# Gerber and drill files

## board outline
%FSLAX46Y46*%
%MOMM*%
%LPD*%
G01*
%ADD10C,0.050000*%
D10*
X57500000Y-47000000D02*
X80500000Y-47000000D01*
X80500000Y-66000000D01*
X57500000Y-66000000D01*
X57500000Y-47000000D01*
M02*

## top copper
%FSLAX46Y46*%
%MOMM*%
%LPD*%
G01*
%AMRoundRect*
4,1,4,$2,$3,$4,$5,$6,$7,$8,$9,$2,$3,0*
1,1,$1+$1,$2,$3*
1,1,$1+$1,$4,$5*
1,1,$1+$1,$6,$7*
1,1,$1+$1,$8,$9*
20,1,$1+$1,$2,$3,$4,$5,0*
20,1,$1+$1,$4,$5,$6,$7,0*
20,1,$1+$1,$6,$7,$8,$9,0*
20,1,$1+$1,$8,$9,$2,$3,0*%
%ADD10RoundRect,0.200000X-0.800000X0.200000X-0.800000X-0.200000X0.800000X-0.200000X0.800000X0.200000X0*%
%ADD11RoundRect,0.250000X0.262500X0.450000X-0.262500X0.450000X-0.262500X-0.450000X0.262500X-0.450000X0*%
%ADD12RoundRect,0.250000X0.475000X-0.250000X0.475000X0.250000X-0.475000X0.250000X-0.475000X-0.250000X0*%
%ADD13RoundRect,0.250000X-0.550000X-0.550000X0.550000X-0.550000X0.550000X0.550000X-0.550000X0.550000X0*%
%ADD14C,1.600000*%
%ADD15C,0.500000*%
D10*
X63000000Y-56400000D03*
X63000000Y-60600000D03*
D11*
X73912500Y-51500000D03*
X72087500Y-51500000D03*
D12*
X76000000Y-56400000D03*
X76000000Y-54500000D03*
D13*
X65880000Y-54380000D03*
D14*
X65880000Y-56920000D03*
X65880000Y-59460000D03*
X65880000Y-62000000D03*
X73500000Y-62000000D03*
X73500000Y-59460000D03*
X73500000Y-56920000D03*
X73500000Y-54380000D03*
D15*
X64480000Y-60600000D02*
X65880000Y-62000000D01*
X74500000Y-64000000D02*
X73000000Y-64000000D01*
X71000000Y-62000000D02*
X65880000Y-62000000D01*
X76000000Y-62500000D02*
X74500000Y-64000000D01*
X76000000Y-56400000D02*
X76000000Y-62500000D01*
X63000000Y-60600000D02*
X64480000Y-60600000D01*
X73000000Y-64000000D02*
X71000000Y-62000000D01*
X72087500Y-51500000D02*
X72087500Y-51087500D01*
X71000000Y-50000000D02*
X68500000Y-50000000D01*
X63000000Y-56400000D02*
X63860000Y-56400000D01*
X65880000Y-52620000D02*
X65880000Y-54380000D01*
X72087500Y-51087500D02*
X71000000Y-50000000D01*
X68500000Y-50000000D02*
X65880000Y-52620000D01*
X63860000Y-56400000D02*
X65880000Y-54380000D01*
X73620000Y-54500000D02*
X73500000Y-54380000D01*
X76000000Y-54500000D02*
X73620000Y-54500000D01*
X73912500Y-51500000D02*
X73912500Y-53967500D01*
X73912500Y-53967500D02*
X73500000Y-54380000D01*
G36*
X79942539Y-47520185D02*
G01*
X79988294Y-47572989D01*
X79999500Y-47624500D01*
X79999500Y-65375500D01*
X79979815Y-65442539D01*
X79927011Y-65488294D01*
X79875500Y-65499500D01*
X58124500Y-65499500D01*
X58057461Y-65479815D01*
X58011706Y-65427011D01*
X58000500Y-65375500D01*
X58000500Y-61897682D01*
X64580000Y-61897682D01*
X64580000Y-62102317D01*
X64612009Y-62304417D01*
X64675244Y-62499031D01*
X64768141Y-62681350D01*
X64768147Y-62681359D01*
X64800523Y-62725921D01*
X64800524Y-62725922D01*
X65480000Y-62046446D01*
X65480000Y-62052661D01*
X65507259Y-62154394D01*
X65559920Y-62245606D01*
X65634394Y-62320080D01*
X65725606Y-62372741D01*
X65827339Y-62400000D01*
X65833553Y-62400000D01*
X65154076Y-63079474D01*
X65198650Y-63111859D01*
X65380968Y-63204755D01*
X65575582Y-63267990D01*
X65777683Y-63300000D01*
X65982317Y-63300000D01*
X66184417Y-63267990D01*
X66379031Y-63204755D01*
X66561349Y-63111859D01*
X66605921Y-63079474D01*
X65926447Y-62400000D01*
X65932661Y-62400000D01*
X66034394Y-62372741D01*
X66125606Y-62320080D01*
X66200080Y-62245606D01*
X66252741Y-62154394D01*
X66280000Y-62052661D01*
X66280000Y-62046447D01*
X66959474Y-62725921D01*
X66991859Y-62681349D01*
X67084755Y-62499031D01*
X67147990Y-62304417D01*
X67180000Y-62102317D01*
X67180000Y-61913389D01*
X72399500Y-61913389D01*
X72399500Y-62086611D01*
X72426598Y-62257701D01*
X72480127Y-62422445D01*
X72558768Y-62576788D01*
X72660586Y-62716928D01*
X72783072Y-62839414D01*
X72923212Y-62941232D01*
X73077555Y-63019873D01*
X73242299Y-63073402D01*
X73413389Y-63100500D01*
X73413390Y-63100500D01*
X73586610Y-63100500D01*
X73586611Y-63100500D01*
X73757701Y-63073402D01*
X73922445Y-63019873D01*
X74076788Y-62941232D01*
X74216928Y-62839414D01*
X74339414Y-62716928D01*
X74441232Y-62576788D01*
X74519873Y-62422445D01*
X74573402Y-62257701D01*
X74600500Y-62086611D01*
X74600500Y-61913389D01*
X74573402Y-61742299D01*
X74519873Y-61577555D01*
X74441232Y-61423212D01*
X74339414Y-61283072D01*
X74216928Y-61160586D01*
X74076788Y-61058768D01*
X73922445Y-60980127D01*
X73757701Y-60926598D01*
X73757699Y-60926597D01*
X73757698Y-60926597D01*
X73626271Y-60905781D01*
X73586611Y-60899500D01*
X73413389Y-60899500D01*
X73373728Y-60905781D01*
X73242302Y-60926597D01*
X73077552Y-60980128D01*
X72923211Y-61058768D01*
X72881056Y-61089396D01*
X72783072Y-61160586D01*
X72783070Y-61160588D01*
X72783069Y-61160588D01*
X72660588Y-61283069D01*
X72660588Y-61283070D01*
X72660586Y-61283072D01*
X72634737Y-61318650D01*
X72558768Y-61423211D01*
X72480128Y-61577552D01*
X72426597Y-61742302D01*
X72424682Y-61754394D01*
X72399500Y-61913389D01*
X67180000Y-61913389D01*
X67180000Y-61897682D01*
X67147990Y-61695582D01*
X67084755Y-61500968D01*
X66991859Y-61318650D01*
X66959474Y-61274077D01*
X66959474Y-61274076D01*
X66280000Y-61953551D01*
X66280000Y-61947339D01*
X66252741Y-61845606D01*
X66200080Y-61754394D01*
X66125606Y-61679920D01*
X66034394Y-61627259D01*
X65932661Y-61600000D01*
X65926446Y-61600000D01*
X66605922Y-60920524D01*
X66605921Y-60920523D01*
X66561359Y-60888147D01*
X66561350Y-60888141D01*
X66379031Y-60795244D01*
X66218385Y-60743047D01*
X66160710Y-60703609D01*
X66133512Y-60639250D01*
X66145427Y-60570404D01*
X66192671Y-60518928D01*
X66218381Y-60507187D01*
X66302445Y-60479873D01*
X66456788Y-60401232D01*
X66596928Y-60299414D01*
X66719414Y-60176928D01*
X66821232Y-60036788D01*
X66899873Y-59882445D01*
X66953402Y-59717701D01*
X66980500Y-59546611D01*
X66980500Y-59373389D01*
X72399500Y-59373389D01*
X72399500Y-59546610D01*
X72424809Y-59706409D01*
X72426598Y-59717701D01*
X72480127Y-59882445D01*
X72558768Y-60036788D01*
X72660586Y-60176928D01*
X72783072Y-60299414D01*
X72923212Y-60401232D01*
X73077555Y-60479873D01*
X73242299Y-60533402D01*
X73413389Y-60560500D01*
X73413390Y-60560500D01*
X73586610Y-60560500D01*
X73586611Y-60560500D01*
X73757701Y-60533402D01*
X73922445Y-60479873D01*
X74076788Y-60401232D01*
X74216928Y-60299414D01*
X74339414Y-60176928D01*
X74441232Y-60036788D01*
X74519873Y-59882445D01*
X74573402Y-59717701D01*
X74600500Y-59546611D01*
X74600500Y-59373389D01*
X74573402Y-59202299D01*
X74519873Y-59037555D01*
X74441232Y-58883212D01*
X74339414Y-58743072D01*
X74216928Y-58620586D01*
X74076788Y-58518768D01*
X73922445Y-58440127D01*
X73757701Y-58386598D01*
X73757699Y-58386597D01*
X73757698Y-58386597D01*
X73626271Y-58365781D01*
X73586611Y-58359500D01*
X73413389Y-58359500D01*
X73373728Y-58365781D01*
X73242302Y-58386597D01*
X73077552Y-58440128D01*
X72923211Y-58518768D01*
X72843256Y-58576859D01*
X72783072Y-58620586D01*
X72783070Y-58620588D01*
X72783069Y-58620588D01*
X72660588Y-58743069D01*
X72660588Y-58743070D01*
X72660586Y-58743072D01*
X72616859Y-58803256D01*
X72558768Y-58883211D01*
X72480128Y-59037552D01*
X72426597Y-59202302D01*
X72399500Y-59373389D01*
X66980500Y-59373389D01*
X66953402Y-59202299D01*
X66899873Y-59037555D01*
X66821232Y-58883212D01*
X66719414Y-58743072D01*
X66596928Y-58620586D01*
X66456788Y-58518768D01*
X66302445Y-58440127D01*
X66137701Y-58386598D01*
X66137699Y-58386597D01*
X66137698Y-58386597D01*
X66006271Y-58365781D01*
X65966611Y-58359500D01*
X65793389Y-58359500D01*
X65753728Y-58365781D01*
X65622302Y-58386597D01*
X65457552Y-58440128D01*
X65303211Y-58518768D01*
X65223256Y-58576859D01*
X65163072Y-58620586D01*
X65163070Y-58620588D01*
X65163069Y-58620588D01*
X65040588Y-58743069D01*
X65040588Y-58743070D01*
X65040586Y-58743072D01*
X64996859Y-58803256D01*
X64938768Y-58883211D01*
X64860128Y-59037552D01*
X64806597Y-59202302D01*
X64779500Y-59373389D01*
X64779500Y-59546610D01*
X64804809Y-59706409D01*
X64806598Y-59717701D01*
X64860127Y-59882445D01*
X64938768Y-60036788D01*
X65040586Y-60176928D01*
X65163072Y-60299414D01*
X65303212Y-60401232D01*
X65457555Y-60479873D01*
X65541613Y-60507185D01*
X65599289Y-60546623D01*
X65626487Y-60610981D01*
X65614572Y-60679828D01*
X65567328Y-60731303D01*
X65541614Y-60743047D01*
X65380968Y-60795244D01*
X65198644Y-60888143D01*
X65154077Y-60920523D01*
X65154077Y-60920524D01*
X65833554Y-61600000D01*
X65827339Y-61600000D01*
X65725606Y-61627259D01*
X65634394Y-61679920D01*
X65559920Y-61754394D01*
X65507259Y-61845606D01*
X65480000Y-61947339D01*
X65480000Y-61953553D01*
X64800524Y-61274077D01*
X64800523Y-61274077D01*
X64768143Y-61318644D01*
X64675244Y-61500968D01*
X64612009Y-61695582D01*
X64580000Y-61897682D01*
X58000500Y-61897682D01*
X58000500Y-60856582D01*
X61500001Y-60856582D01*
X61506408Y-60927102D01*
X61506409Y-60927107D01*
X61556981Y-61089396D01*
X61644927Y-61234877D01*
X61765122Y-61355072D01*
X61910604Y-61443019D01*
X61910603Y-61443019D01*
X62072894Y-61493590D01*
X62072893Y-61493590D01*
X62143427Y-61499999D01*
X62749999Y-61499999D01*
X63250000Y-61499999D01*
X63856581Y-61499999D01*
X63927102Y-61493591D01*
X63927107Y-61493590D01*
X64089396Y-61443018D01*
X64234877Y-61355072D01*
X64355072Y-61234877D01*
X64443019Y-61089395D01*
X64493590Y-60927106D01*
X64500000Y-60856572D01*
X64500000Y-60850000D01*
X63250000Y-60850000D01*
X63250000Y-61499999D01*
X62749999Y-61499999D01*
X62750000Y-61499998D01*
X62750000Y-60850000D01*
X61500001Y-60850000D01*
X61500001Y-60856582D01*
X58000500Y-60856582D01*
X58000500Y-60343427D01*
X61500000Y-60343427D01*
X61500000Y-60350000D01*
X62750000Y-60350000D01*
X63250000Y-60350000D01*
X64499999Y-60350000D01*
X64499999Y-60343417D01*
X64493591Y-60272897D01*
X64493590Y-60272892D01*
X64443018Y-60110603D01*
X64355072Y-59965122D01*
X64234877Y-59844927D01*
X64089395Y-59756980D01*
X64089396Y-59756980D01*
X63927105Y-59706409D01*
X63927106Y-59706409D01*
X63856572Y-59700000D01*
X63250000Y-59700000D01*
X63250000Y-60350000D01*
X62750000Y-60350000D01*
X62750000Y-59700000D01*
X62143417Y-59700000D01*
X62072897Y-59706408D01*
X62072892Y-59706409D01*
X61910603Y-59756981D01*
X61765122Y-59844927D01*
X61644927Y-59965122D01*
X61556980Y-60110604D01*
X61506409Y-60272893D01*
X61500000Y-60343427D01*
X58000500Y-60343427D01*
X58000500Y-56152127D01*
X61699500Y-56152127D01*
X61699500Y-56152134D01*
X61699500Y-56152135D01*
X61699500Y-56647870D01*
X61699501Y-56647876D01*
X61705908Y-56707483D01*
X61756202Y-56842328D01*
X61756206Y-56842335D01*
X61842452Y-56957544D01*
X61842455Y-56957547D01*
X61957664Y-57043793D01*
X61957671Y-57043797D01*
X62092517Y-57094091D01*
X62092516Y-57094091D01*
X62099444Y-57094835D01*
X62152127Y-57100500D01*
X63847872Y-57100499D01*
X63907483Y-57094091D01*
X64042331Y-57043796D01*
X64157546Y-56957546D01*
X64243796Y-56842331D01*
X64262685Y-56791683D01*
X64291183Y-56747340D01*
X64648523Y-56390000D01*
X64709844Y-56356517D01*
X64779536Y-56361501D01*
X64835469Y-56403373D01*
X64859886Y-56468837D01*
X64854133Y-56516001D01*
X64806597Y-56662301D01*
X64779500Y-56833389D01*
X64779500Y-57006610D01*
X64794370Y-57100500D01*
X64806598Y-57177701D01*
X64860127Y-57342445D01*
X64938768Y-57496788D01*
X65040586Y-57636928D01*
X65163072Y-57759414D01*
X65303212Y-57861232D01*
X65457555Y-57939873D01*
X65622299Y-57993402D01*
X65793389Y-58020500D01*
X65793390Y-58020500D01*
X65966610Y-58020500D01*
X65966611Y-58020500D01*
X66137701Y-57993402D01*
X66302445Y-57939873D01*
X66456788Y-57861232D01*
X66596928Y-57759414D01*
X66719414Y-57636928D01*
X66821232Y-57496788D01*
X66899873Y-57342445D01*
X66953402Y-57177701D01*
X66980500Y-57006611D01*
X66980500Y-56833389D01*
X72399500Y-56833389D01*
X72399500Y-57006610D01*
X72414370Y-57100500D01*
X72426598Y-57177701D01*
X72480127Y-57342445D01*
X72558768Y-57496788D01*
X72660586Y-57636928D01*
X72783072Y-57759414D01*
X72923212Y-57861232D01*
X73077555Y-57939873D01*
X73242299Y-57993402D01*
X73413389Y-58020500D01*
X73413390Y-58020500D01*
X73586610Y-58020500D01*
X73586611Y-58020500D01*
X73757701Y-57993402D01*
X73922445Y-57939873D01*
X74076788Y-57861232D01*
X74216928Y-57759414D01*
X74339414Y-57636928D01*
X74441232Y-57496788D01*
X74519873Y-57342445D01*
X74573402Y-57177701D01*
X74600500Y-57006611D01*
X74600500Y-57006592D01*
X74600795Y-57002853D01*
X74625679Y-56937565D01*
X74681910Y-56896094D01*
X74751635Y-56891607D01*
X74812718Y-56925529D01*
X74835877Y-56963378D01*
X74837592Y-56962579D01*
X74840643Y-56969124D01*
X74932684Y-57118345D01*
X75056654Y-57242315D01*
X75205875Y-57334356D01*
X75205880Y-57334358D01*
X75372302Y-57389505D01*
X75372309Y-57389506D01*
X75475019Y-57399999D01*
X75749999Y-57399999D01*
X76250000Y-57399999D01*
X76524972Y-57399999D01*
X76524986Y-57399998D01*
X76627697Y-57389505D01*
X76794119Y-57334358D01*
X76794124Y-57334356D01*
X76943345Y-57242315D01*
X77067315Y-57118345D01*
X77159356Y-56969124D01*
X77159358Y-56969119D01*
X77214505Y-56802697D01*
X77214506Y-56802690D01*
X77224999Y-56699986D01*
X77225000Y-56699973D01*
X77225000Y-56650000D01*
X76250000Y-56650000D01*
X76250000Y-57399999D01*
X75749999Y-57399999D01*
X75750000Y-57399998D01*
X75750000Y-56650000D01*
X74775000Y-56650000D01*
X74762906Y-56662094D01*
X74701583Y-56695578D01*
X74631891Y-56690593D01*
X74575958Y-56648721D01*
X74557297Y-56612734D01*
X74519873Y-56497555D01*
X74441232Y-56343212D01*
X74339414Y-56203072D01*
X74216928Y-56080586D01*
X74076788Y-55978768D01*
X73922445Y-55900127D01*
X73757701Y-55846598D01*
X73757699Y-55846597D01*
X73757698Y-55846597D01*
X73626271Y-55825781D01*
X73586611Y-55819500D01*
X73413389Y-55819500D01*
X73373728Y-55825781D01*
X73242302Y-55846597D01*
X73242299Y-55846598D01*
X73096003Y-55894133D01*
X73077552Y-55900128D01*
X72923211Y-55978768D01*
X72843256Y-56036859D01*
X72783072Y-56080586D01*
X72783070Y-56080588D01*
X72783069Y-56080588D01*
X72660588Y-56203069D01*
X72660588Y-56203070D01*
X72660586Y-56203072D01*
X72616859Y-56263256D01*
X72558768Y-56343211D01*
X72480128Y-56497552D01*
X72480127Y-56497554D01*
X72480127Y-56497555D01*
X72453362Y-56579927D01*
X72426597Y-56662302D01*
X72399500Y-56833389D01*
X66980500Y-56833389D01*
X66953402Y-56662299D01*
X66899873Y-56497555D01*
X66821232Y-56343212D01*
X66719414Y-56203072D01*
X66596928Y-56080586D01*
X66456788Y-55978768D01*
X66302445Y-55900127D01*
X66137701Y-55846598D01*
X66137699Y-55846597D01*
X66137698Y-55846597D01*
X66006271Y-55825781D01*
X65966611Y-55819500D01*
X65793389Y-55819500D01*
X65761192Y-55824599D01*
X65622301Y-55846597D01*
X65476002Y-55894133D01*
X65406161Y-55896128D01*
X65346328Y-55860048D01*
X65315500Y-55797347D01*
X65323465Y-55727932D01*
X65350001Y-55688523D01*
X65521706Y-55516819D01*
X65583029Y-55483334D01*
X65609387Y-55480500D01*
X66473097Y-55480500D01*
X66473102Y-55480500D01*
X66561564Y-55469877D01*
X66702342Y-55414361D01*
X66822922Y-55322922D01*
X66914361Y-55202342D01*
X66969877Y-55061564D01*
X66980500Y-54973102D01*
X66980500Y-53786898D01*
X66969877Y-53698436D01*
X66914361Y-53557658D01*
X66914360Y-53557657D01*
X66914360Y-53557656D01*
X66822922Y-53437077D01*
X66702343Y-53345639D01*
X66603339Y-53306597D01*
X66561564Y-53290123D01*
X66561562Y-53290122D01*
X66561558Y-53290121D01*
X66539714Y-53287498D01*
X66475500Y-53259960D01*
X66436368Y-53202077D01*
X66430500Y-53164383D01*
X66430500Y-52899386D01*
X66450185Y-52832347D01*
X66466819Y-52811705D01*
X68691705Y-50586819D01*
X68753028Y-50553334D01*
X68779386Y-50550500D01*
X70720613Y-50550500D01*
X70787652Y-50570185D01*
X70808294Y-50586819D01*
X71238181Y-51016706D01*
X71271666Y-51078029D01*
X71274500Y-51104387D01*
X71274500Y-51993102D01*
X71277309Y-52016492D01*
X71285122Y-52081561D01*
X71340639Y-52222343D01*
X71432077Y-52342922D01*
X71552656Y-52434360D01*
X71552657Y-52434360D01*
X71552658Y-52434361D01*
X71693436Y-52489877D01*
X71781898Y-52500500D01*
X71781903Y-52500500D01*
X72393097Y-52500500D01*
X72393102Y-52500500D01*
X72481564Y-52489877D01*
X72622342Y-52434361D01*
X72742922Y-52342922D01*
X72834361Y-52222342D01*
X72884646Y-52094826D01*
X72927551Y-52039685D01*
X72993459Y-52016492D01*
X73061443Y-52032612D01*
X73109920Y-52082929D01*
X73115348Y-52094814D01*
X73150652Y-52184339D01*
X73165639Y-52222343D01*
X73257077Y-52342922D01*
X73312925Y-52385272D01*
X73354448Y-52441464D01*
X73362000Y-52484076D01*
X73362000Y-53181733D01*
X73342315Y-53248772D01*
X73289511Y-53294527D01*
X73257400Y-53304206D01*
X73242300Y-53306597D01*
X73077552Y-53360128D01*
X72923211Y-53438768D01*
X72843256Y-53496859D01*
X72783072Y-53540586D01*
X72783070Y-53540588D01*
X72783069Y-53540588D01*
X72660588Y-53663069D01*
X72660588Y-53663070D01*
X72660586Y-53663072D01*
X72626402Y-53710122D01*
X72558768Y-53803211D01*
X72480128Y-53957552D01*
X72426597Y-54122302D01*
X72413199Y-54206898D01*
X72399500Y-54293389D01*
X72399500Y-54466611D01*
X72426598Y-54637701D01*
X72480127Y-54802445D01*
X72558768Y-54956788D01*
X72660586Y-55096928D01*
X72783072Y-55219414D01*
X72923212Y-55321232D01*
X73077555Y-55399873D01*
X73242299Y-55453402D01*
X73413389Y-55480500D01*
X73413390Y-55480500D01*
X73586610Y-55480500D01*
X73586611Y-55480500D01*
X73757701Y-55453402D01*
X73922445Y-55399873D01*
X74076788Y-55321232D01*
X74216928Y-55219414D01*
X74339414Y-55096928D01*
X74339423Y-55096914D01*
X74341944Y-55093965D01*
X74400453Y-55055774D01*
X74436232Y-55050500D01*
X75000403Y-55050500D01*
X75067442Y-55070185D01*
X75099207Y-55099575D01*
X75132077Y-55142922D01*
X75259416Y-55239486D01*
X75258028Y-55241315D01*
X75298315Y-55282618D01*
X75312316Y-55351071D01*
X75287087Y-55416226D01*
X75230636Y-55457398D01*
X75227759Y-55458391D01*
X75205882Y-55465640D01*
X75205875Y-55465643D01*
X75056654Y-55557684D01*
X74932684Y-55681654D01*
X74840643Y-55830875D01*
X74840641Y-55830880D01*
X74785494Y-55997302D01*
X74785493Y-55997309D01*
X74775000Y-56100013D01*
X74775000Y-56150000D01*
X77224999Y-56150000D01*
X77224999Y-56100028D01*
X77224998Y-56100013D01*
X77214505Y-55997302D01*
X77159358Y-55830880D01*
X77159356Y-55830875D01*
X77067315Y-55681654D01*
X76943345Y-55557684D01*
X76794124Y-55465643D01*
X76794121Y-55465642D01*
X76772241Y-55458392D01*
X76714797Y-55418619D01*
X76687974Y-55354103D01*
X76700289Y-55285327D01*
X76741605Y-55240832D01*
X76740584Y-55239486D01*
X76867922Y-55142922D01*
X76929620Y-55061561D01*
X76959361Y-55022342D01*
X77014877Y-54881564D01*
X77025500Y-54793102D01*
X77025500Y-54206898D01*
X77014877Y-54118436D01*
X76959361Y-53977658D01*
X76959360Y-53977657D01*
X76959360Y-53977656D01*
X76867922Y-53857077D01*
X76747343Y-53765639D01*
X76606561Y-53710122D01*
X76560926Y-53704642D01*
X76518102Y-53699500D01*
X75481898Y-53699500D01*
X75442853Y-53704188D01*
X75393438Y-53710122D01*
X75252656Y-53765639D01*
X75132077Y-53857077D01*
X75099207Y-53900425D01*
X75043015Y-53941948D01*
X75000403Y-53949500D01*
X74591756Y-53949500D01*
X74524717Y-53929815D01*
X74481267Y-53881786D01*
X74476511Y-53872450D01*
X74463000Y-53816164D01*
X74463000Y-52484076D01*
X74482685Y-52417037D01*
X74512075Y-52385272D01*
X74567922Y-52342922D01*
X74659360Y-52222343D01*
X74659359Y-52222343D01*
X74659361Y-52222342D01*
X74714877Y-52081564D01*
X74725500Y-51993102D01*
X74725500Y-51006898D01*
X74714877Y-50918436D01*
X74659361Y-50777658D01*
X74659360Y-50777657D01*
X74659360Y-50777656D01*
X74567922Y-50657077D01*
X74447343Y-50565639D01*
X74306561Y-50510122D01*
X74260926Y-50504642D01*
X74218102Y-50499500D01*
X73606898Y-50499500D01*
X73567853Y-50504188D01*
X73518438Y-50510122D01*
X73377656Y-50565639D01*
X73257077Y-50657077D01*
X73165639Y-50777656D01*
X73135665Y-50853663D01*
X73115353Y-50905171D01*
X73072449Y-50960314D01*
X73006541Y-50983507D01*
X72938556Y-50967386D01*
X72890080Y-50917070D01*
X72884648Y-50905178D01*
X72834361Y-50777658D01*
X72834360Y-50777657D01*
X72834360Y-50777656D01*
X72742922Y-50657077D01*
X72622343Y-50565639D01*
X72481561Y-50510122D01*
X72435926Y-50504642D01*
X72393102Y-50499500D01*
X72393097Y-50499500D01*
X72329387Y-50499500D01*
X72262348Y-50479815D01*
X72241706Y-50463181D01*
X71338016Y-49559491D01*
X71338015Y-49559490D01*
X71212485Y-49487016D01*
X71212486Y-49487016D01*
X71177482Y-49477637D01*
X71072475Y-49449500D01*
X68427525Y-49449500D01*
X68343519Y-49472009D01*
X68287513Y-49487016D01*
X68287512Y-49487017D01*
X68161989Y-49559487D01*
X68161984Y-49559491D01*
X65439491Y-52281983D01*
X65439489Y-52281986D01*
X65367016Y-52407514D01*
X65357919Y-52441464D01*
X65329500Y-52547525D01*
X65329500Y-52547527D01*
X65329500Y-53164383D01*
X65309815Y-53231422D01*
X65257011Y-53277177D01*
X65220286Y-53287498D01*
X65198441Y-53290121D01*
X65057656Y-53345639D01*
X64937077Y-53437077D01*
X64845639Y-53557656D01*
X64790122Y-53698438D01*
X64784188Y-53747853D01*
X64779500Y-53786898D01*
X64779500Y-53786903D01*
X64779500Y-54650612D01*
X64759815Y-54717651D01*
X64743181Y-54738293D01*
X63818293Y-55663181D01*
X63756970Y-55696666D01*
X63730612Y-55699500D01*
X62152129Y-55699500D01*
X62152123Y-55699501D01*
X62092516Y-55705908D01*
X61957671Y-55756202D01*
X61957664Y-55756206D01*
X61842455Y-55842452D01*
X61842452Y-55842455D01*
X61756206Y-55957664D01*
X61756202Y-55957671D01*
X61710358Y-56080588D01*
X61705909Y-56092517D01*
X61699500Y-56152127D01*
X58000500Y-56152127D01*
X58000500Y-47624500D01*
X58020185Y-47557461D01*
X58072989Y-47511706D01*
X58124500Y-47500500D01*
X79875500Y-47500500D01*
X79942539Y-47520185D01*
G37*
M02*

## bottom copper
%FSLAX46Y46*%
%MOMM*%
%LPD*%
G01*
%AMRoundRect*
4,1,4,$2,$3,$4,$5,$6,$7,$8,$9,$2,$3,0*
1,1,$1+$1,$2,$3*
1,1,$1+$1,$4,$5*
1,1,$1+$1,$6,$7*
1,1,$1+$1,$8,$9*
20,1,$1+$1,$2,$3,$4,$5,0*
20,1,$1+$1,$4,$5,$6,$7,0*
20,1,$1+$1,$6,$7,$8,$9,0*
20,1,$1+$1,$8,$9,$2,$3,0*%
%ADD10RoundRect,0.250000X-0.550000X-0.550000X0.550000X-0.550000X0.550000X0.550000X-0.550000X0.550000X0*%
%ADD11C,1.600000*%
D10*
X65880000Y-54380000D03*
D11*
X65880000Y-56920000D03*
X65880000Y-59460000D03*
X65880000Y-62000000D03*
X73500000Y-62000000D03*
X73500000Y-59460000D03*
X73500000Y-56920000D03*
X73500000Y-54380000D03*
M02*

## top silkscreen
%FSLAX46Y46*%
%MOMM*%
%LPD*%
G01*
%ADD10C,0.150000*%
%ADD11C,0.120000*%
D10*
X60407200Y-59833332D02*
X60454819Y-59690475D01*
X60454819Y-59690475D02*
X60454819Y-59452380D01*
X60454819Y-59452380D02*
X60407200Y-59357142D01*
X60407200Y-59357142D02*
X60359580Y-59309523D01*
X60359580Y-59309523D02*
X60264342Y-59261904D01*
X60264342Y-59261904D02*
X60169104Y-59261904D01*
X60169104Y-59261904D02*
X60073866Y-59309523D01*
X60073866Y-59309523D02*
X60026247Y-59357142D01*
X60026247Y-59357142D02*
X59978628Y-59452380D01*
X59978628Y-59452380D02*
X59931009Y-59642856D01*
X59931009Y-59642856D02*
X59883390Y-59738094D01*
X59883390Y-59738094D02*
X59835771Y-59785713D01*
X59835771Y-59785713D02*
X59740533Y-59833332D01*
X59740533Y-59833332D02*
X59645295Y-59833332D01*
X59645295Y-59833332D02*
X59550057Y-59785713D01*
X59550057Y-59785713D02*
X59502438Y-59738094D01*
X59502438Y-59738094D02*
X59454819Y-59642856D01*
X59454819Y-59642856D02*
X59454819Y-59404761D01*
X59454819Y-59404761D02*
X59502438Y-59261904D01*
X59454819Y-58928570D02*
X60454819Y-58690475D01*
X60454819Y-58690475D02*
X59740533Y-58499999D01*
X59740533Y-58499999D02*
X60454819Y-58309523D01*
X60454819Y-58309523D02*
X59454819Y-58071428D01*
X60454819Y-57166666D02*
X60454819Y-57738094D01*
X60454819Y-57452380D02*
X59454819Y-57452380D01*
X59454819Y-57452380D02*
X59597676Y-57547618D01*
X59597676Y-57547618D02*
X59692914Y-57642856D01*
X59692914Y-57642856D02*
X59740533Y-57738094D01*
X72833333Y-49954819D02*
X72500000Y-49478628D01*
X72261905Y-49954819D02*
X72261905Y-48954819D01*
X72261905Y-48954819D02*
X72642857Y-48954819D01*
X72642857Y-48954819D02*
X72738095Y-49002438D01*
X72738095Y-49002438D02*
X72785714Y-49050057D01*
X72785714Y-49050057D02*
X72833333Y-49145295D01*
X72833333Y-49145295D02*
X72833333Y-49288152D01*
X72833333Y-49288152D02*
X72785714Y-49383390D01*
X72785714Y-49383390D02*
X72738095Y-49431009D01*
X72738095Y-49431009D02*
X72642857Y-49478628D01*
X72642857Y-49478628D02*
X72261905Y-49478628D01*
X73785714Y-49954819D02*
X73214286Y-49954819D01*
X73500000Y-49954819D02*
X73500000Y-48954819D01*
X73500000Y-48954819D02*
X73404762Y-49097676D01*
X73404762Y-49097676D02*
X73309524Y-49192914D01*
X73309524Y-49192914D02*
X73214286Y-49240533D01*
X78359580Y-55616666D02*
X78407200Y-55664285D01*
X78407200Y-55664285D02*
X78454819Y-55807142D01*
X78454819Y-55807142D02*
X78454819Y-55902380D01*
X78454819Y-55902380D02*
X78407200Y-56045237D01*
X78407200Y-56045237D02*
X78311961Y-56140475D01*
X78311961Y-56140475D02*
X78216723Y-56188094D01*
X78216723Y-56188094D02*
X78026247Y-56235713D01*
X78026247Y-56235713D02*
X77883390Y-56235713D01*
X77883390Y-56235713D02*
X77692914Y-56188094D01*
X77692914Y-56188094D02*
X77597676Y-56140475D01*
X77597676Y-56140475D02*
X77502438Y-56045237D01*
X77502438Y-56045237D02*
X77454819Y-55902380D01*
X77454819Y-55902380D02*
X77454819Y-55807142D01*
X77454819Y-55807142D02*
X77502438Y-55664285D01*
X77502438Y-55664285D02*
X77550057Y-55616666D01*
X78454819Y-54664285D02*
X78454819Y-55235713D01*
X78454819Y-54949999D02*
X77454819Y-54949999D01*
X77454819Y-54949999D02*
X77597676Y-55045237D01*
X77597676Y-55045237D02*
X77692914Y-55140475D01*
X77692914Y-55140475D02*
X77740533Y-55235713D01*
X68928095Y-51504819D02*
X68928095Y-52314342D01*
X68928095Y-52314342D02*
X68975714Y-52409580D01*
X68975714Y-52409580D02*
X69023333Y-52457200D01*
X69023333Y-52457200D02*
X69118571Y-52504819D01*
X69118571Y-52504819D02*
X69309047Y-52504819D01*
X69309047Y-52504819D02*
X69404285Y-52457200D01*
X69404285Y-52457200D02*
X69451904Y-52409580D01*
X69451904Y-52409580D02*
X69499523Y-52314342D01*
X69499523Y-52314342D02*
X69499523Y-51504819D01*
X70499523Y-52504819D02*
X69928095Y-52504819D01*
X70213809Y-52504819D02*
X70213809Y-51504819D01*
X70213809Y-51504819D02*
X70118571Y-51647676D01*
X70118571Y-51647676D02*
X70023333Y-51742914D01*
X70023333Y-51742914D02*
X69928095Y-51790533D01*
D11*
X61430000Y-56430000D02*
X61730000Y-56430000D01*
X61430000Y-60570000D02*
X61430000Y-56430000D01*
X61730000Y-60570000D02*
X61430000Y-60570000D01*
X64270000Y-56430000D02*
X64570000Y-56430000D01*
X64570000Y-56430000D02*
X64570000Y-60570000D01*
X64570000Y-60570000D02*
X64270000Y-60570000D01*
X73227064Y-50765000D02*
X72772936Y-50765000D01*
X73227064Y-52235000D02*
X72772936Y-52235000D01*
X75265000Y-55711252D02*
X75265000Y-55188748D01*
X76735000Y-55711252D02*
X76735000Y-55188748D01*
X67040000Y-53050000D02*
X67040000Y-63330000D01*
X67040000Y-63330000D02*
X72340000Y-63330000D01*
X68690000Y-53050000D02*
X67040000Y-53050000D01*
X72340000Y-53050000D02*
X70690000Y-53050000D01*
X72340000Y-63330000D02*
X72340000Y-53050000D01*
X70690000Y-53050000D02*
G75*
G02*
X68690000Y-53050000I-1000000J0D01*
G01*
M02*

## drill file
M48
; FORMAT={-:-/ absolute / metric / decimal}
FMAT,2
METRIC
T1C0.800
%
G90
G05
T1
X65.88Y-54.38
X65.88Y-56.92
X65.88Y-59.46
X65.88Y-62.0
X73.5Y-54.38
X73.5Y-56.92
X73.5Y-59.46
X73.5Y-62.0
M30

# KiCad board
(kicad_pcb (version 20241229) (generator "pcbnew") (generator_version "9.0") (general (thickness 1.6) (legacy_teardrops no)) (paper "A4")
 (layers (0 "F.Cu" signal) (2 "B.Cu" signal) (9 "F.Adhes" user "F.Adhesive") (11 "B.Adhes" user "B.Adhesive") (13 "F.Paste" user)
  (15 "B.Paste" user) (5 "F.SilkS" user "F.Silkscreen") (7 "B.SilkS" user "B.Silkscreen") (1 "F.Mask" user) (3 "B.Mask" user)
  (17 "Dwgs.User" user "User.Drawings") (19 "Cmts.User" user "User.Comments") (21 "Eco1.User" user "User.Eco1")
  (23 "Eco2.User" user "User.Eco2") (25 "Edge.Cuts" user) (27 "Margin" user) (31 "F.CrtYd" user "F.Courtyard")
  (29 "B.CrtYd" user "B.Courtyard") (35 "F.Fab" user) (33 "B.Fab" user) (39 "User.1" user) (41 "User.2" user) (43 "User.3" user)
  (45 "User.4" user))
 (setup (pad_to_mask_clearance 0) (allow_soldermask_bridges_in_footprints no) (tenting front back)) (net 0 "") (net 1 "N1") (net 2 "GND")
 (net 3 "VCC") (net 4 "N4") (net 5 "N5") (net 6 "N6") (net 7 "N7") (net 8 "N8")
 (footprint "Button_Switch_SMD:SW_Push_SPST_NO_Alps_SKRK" (layer "F.Cu") (at 63 58.5 -90)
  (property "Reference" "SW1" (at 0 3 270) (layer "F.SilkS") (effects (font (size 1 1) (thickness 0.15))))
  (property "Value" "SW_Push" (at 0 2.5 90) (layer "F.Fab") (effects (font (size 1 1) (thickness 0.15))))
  (fp_line (start -2.07 1.57) (end -2.07 1.27) (stroke (width 0.12) (type solid)) (layer "F.SilkS"))
  (fp_line (start 2.07 1.57) (end -2.07 1.57) (stroke (width 0.12) (type solid)) (layer "F.SilkS"))
  (fp_line (start 2.07 1.27) (end 2.07 1.57) (stroke (width 0.12) (type solid)) (layer "F.SilkS"))
  (fp_line (start -2.07 -1.27) (end -2.07 -1.57) (stroke (width 0.12) (type solid)) (layer "F.SilkS"))
  (fp_line (start -2.07 -1.57) (end 2.07 -1.57) (stroke (width 0.12) (type solid)) (layer "F.SilkS"))
  (fp_line (start 2.07 -1.57) (end 2.07 -1.27) (stroke (width 0.12) (type solid)) (layer "F.SilkS"))
  (pad "1" smd roundrect (at -2.1 0 270) (size 0.8 2) (layers "F.Cu" "F.Mask" "F.Paste") (roundrect_rratio 0.25) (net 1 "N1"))
  (pad "2" smd roundrect (at 2.1 0 270) (size 0.8 2) (layers "F.Cu" "F.Mask" "F.Paste") (roundrect_rratio 0.25) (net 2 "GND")))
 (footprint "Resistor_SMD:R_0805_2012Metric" (layer "F.Cu") (at 73 51.5 180)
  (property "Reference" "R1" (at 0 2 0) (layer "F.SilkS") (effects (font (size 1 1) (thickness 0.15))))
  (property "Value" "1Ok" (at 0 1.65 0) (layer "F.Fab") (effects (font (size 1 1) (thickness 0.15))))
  (fp_line (start -0.227064 0.735) (end 0.227064 0.735) (stroke (width 0.12) (type solid)) (layer "F.SilkS"))
  (fp_line (start -0.227064 -0.735) (end 0.227064 -0.735) (stroke (width 0.12) (type solid)) (layer "F.SilkS"))
  (pad "1" smd roundrect (at -0.9125 0 180) (size 1.025 1.4) (layers "F.Cu" "F.Mask" "F.Paste") (roundrect_rratio 0.243902) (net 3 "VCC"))
  (pad "2" smd roundrect (at 0.9125 0 180) (size 1.025 1.4) (layers "F.Cu" "F.Mask" "F.Paste") (roundrect_rratio 0.243902) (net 1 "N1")))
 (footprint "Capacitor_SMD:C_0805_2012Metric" (layer "F.Cu") (at 76 55.45 90)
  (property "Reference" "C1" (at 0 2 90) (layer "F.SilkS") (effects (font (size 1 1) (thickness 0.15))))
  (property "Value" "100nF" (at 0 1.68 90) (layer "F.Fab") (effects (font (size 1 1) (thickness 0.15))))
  (fp_line (start -0.261252 -0.735) (end 0.261252 -0.735) (stroke (width 0.12) (type solid)) (layer "F.SilkS"))
  (fp_line (start -0.261252 0.735) (end 0.261252 0.735) (stroke (width 0.12) (type solid)) (layer "F.SilkS"))
  (pad "1" smd roundrect (at -0.95 0 90) (size 1 1.45) (layers "F.Cu" "F.Mask" "F.Paste") (roundrect_rratio 0.25) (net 2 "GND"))
  (pad "2" smd roundrect (at 0.95 0 90) (size 1 1.45) (layers "F.Cu" "F.Mask" "F.Paste") (roundrect_rratio 0.25) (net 3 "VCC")))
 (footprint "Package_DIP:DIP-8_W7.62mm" (layer "F.Cu") (at 65.88 54.38)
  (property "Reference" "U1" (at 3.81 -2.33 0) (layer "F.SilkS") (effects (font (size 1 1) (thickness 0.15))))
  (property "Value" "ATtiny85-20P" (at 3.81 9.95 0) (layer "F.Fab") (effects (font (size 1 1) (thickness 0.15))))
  (fp_line (start 1.16 -1.33) (end 1.16 8.95) (stroke (width 0.12) (type solid)) (layer "F.SilkS"))
  (fp_line (start 1.16 8.95) (end 6.46 8.95) (stroke (width 0.12) (type solid)) (layer "F.SilkS"))
  (fp_line (start 2.81 -1.33) (end 1.16 -1.33) (stroke (width 0.12) (type solid)) (layer "F.SilkS"))
  (fp_line (start 6.46 -1.33) (end 4.81 -1.33) (stroke (width 0.12) (type solid)) (layer "F.SilkS"))
  (fp_line (start 6.46 8.95) (end 6.46 -1.33) (stroke (width 0.12) (type solid)) (layer "F.SilkS"))
  (fp_arc (start 4.81 -1.33) (mid 3.81 -0.33) (end 2.81 -1.33) (stroke (width 0.12) (type solid)) (layer "F.SilkS"))
  (pad "1" thru_hole roundrect (at 0 0) (size 1.6 1.6) (drill 0.8) (layers "*.Cu" "*.Mask") (remove_unused_layers no)
   (roundrect_rratio 0.15625) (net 1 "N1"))
  (pad "2" thru_hole circle (at 0 2.54) (size 1.6 1.6) (drill 0.8) (layers "*.Cu" "*.Mask") (remove_unused_layers no) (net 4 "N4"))
  (pad "3" thru_hole circle (at 0 5.08) (size 1.6 1.6) (drill 0.8) (layers "*.Cu" "*.Mask") (remove_unused_layers no) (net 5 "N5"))
  (pad "4" thru_hole circle (at 0 7.62) (size 1.6 1.6) (drill 0.8) (layers "*.Cu" "*.Mask") (remove_unused_layers no) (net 2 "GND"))
  (pad "5" thru_hole circle (at 7.62 7.62) (size 1.6 1.6) (drill 0.8) (layers "*.Cu" "*.Mask") (remove_unused_layers no) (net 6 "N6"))
  (pad "6" thru_hole circle (at 7.62 5.08) (size 1.6 1.6) (drill 0.8) (layers "*.Cu" "*.Mask") (remove_unused_layers no) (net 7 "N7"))
  (pad "7" thru_hole circle (at 7.62 2.54) (size 1.6 1.6) (drill 0.8) (layers "*.Cu" "*.Mask") (remove_unused_layers no) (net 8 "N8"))
  (pad "8" thru_hole circle (at 7.62 0) (size 1.6 1.6) (drill 0.8) (layers "*.Cu" "*.Mask") (remove_unused_layers no) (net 3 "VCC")))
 (gr_rect (start 57.5 47) (end 80.5 66) (stroke (width 0.05) (type solid)) (fill no) (layer "Edge.Cuts"))
 (segment (start 64.48 60.6) (end 65.88 62) (width 0.5) (layer "F.Cu") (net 2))
 (segment (start 74.5 64) (end 73 64) (width 0.5) (layer "F.Cu") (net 2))
 (segment (start 71 62) (end 65.88 62) (width 0.5) (layer "F.Cu") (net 2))
 (segment (start 76 62.5) (end 74.5 64) (width 0.5) (layer "F.Cu") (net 2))
 (segment (start 76 56.4) (end 76 62.5) (width 0.5) (layer "F.Cu") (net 2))
 (segment (start 63 60.6) (end 64.48 60.6) (width 0.5) (layer "F.Cu") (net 2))
 (segment (start 73 64) (end 71 62) (width 0.5) (layer "F.Cu") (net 2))
 (segment (start 72.0875 51.5) (end 72.0875 51.0875) (width 0.5) (layer "F.Cu") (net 1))
 (segment (start 71 50) (end 68.5 50) (width 0.5) (layer "F.Cu") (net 1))
 (segment (start 63 56.4) (end 63.86 56.4) (width 0.5) (layer "F.Cu") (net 1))
 (segment (start 65.88 52.62) (end 65.88 54.38) (width 0.5) (layer "F.Cu") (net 1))
 (segment (start 72.0875 51.0875) (end 71 50) (width 0.5) (layer "F.Cu") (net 1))
 (segment (start 68.5 50) (end 65.88 52.62) (width 0.5) (layer "F.Cu") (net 1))
 (segment (start 63.86 56.4) (end 65.88 54.38) (width 0.5) (layer "F.Cu") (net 1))
 (segment (start 73.62 54.5) (end 73.5 54.38) (width 0.5) (layer "F.Cu") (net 3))
 (segment (start 76 54.5) (end 73.62 54.5) (width 0.5) (layer "F.Cu") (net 3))
 (segment (start 73.9125 51.5) (end 73.9125 53.9675) (width 0.5) (layer "F.Cu") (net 3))
 (segment (start 73.9125 53.9675) (end 73.5 54.38) (width 0.5) (layer "F.Cu") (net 3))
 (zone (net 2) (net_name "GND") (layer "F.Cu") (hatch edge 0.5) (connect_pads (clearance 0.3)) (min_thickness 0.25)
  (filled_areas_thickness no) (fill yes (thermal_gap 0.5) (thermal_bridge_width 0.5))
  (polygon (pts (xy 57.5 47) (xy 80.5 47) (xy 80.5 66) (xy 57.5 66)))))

